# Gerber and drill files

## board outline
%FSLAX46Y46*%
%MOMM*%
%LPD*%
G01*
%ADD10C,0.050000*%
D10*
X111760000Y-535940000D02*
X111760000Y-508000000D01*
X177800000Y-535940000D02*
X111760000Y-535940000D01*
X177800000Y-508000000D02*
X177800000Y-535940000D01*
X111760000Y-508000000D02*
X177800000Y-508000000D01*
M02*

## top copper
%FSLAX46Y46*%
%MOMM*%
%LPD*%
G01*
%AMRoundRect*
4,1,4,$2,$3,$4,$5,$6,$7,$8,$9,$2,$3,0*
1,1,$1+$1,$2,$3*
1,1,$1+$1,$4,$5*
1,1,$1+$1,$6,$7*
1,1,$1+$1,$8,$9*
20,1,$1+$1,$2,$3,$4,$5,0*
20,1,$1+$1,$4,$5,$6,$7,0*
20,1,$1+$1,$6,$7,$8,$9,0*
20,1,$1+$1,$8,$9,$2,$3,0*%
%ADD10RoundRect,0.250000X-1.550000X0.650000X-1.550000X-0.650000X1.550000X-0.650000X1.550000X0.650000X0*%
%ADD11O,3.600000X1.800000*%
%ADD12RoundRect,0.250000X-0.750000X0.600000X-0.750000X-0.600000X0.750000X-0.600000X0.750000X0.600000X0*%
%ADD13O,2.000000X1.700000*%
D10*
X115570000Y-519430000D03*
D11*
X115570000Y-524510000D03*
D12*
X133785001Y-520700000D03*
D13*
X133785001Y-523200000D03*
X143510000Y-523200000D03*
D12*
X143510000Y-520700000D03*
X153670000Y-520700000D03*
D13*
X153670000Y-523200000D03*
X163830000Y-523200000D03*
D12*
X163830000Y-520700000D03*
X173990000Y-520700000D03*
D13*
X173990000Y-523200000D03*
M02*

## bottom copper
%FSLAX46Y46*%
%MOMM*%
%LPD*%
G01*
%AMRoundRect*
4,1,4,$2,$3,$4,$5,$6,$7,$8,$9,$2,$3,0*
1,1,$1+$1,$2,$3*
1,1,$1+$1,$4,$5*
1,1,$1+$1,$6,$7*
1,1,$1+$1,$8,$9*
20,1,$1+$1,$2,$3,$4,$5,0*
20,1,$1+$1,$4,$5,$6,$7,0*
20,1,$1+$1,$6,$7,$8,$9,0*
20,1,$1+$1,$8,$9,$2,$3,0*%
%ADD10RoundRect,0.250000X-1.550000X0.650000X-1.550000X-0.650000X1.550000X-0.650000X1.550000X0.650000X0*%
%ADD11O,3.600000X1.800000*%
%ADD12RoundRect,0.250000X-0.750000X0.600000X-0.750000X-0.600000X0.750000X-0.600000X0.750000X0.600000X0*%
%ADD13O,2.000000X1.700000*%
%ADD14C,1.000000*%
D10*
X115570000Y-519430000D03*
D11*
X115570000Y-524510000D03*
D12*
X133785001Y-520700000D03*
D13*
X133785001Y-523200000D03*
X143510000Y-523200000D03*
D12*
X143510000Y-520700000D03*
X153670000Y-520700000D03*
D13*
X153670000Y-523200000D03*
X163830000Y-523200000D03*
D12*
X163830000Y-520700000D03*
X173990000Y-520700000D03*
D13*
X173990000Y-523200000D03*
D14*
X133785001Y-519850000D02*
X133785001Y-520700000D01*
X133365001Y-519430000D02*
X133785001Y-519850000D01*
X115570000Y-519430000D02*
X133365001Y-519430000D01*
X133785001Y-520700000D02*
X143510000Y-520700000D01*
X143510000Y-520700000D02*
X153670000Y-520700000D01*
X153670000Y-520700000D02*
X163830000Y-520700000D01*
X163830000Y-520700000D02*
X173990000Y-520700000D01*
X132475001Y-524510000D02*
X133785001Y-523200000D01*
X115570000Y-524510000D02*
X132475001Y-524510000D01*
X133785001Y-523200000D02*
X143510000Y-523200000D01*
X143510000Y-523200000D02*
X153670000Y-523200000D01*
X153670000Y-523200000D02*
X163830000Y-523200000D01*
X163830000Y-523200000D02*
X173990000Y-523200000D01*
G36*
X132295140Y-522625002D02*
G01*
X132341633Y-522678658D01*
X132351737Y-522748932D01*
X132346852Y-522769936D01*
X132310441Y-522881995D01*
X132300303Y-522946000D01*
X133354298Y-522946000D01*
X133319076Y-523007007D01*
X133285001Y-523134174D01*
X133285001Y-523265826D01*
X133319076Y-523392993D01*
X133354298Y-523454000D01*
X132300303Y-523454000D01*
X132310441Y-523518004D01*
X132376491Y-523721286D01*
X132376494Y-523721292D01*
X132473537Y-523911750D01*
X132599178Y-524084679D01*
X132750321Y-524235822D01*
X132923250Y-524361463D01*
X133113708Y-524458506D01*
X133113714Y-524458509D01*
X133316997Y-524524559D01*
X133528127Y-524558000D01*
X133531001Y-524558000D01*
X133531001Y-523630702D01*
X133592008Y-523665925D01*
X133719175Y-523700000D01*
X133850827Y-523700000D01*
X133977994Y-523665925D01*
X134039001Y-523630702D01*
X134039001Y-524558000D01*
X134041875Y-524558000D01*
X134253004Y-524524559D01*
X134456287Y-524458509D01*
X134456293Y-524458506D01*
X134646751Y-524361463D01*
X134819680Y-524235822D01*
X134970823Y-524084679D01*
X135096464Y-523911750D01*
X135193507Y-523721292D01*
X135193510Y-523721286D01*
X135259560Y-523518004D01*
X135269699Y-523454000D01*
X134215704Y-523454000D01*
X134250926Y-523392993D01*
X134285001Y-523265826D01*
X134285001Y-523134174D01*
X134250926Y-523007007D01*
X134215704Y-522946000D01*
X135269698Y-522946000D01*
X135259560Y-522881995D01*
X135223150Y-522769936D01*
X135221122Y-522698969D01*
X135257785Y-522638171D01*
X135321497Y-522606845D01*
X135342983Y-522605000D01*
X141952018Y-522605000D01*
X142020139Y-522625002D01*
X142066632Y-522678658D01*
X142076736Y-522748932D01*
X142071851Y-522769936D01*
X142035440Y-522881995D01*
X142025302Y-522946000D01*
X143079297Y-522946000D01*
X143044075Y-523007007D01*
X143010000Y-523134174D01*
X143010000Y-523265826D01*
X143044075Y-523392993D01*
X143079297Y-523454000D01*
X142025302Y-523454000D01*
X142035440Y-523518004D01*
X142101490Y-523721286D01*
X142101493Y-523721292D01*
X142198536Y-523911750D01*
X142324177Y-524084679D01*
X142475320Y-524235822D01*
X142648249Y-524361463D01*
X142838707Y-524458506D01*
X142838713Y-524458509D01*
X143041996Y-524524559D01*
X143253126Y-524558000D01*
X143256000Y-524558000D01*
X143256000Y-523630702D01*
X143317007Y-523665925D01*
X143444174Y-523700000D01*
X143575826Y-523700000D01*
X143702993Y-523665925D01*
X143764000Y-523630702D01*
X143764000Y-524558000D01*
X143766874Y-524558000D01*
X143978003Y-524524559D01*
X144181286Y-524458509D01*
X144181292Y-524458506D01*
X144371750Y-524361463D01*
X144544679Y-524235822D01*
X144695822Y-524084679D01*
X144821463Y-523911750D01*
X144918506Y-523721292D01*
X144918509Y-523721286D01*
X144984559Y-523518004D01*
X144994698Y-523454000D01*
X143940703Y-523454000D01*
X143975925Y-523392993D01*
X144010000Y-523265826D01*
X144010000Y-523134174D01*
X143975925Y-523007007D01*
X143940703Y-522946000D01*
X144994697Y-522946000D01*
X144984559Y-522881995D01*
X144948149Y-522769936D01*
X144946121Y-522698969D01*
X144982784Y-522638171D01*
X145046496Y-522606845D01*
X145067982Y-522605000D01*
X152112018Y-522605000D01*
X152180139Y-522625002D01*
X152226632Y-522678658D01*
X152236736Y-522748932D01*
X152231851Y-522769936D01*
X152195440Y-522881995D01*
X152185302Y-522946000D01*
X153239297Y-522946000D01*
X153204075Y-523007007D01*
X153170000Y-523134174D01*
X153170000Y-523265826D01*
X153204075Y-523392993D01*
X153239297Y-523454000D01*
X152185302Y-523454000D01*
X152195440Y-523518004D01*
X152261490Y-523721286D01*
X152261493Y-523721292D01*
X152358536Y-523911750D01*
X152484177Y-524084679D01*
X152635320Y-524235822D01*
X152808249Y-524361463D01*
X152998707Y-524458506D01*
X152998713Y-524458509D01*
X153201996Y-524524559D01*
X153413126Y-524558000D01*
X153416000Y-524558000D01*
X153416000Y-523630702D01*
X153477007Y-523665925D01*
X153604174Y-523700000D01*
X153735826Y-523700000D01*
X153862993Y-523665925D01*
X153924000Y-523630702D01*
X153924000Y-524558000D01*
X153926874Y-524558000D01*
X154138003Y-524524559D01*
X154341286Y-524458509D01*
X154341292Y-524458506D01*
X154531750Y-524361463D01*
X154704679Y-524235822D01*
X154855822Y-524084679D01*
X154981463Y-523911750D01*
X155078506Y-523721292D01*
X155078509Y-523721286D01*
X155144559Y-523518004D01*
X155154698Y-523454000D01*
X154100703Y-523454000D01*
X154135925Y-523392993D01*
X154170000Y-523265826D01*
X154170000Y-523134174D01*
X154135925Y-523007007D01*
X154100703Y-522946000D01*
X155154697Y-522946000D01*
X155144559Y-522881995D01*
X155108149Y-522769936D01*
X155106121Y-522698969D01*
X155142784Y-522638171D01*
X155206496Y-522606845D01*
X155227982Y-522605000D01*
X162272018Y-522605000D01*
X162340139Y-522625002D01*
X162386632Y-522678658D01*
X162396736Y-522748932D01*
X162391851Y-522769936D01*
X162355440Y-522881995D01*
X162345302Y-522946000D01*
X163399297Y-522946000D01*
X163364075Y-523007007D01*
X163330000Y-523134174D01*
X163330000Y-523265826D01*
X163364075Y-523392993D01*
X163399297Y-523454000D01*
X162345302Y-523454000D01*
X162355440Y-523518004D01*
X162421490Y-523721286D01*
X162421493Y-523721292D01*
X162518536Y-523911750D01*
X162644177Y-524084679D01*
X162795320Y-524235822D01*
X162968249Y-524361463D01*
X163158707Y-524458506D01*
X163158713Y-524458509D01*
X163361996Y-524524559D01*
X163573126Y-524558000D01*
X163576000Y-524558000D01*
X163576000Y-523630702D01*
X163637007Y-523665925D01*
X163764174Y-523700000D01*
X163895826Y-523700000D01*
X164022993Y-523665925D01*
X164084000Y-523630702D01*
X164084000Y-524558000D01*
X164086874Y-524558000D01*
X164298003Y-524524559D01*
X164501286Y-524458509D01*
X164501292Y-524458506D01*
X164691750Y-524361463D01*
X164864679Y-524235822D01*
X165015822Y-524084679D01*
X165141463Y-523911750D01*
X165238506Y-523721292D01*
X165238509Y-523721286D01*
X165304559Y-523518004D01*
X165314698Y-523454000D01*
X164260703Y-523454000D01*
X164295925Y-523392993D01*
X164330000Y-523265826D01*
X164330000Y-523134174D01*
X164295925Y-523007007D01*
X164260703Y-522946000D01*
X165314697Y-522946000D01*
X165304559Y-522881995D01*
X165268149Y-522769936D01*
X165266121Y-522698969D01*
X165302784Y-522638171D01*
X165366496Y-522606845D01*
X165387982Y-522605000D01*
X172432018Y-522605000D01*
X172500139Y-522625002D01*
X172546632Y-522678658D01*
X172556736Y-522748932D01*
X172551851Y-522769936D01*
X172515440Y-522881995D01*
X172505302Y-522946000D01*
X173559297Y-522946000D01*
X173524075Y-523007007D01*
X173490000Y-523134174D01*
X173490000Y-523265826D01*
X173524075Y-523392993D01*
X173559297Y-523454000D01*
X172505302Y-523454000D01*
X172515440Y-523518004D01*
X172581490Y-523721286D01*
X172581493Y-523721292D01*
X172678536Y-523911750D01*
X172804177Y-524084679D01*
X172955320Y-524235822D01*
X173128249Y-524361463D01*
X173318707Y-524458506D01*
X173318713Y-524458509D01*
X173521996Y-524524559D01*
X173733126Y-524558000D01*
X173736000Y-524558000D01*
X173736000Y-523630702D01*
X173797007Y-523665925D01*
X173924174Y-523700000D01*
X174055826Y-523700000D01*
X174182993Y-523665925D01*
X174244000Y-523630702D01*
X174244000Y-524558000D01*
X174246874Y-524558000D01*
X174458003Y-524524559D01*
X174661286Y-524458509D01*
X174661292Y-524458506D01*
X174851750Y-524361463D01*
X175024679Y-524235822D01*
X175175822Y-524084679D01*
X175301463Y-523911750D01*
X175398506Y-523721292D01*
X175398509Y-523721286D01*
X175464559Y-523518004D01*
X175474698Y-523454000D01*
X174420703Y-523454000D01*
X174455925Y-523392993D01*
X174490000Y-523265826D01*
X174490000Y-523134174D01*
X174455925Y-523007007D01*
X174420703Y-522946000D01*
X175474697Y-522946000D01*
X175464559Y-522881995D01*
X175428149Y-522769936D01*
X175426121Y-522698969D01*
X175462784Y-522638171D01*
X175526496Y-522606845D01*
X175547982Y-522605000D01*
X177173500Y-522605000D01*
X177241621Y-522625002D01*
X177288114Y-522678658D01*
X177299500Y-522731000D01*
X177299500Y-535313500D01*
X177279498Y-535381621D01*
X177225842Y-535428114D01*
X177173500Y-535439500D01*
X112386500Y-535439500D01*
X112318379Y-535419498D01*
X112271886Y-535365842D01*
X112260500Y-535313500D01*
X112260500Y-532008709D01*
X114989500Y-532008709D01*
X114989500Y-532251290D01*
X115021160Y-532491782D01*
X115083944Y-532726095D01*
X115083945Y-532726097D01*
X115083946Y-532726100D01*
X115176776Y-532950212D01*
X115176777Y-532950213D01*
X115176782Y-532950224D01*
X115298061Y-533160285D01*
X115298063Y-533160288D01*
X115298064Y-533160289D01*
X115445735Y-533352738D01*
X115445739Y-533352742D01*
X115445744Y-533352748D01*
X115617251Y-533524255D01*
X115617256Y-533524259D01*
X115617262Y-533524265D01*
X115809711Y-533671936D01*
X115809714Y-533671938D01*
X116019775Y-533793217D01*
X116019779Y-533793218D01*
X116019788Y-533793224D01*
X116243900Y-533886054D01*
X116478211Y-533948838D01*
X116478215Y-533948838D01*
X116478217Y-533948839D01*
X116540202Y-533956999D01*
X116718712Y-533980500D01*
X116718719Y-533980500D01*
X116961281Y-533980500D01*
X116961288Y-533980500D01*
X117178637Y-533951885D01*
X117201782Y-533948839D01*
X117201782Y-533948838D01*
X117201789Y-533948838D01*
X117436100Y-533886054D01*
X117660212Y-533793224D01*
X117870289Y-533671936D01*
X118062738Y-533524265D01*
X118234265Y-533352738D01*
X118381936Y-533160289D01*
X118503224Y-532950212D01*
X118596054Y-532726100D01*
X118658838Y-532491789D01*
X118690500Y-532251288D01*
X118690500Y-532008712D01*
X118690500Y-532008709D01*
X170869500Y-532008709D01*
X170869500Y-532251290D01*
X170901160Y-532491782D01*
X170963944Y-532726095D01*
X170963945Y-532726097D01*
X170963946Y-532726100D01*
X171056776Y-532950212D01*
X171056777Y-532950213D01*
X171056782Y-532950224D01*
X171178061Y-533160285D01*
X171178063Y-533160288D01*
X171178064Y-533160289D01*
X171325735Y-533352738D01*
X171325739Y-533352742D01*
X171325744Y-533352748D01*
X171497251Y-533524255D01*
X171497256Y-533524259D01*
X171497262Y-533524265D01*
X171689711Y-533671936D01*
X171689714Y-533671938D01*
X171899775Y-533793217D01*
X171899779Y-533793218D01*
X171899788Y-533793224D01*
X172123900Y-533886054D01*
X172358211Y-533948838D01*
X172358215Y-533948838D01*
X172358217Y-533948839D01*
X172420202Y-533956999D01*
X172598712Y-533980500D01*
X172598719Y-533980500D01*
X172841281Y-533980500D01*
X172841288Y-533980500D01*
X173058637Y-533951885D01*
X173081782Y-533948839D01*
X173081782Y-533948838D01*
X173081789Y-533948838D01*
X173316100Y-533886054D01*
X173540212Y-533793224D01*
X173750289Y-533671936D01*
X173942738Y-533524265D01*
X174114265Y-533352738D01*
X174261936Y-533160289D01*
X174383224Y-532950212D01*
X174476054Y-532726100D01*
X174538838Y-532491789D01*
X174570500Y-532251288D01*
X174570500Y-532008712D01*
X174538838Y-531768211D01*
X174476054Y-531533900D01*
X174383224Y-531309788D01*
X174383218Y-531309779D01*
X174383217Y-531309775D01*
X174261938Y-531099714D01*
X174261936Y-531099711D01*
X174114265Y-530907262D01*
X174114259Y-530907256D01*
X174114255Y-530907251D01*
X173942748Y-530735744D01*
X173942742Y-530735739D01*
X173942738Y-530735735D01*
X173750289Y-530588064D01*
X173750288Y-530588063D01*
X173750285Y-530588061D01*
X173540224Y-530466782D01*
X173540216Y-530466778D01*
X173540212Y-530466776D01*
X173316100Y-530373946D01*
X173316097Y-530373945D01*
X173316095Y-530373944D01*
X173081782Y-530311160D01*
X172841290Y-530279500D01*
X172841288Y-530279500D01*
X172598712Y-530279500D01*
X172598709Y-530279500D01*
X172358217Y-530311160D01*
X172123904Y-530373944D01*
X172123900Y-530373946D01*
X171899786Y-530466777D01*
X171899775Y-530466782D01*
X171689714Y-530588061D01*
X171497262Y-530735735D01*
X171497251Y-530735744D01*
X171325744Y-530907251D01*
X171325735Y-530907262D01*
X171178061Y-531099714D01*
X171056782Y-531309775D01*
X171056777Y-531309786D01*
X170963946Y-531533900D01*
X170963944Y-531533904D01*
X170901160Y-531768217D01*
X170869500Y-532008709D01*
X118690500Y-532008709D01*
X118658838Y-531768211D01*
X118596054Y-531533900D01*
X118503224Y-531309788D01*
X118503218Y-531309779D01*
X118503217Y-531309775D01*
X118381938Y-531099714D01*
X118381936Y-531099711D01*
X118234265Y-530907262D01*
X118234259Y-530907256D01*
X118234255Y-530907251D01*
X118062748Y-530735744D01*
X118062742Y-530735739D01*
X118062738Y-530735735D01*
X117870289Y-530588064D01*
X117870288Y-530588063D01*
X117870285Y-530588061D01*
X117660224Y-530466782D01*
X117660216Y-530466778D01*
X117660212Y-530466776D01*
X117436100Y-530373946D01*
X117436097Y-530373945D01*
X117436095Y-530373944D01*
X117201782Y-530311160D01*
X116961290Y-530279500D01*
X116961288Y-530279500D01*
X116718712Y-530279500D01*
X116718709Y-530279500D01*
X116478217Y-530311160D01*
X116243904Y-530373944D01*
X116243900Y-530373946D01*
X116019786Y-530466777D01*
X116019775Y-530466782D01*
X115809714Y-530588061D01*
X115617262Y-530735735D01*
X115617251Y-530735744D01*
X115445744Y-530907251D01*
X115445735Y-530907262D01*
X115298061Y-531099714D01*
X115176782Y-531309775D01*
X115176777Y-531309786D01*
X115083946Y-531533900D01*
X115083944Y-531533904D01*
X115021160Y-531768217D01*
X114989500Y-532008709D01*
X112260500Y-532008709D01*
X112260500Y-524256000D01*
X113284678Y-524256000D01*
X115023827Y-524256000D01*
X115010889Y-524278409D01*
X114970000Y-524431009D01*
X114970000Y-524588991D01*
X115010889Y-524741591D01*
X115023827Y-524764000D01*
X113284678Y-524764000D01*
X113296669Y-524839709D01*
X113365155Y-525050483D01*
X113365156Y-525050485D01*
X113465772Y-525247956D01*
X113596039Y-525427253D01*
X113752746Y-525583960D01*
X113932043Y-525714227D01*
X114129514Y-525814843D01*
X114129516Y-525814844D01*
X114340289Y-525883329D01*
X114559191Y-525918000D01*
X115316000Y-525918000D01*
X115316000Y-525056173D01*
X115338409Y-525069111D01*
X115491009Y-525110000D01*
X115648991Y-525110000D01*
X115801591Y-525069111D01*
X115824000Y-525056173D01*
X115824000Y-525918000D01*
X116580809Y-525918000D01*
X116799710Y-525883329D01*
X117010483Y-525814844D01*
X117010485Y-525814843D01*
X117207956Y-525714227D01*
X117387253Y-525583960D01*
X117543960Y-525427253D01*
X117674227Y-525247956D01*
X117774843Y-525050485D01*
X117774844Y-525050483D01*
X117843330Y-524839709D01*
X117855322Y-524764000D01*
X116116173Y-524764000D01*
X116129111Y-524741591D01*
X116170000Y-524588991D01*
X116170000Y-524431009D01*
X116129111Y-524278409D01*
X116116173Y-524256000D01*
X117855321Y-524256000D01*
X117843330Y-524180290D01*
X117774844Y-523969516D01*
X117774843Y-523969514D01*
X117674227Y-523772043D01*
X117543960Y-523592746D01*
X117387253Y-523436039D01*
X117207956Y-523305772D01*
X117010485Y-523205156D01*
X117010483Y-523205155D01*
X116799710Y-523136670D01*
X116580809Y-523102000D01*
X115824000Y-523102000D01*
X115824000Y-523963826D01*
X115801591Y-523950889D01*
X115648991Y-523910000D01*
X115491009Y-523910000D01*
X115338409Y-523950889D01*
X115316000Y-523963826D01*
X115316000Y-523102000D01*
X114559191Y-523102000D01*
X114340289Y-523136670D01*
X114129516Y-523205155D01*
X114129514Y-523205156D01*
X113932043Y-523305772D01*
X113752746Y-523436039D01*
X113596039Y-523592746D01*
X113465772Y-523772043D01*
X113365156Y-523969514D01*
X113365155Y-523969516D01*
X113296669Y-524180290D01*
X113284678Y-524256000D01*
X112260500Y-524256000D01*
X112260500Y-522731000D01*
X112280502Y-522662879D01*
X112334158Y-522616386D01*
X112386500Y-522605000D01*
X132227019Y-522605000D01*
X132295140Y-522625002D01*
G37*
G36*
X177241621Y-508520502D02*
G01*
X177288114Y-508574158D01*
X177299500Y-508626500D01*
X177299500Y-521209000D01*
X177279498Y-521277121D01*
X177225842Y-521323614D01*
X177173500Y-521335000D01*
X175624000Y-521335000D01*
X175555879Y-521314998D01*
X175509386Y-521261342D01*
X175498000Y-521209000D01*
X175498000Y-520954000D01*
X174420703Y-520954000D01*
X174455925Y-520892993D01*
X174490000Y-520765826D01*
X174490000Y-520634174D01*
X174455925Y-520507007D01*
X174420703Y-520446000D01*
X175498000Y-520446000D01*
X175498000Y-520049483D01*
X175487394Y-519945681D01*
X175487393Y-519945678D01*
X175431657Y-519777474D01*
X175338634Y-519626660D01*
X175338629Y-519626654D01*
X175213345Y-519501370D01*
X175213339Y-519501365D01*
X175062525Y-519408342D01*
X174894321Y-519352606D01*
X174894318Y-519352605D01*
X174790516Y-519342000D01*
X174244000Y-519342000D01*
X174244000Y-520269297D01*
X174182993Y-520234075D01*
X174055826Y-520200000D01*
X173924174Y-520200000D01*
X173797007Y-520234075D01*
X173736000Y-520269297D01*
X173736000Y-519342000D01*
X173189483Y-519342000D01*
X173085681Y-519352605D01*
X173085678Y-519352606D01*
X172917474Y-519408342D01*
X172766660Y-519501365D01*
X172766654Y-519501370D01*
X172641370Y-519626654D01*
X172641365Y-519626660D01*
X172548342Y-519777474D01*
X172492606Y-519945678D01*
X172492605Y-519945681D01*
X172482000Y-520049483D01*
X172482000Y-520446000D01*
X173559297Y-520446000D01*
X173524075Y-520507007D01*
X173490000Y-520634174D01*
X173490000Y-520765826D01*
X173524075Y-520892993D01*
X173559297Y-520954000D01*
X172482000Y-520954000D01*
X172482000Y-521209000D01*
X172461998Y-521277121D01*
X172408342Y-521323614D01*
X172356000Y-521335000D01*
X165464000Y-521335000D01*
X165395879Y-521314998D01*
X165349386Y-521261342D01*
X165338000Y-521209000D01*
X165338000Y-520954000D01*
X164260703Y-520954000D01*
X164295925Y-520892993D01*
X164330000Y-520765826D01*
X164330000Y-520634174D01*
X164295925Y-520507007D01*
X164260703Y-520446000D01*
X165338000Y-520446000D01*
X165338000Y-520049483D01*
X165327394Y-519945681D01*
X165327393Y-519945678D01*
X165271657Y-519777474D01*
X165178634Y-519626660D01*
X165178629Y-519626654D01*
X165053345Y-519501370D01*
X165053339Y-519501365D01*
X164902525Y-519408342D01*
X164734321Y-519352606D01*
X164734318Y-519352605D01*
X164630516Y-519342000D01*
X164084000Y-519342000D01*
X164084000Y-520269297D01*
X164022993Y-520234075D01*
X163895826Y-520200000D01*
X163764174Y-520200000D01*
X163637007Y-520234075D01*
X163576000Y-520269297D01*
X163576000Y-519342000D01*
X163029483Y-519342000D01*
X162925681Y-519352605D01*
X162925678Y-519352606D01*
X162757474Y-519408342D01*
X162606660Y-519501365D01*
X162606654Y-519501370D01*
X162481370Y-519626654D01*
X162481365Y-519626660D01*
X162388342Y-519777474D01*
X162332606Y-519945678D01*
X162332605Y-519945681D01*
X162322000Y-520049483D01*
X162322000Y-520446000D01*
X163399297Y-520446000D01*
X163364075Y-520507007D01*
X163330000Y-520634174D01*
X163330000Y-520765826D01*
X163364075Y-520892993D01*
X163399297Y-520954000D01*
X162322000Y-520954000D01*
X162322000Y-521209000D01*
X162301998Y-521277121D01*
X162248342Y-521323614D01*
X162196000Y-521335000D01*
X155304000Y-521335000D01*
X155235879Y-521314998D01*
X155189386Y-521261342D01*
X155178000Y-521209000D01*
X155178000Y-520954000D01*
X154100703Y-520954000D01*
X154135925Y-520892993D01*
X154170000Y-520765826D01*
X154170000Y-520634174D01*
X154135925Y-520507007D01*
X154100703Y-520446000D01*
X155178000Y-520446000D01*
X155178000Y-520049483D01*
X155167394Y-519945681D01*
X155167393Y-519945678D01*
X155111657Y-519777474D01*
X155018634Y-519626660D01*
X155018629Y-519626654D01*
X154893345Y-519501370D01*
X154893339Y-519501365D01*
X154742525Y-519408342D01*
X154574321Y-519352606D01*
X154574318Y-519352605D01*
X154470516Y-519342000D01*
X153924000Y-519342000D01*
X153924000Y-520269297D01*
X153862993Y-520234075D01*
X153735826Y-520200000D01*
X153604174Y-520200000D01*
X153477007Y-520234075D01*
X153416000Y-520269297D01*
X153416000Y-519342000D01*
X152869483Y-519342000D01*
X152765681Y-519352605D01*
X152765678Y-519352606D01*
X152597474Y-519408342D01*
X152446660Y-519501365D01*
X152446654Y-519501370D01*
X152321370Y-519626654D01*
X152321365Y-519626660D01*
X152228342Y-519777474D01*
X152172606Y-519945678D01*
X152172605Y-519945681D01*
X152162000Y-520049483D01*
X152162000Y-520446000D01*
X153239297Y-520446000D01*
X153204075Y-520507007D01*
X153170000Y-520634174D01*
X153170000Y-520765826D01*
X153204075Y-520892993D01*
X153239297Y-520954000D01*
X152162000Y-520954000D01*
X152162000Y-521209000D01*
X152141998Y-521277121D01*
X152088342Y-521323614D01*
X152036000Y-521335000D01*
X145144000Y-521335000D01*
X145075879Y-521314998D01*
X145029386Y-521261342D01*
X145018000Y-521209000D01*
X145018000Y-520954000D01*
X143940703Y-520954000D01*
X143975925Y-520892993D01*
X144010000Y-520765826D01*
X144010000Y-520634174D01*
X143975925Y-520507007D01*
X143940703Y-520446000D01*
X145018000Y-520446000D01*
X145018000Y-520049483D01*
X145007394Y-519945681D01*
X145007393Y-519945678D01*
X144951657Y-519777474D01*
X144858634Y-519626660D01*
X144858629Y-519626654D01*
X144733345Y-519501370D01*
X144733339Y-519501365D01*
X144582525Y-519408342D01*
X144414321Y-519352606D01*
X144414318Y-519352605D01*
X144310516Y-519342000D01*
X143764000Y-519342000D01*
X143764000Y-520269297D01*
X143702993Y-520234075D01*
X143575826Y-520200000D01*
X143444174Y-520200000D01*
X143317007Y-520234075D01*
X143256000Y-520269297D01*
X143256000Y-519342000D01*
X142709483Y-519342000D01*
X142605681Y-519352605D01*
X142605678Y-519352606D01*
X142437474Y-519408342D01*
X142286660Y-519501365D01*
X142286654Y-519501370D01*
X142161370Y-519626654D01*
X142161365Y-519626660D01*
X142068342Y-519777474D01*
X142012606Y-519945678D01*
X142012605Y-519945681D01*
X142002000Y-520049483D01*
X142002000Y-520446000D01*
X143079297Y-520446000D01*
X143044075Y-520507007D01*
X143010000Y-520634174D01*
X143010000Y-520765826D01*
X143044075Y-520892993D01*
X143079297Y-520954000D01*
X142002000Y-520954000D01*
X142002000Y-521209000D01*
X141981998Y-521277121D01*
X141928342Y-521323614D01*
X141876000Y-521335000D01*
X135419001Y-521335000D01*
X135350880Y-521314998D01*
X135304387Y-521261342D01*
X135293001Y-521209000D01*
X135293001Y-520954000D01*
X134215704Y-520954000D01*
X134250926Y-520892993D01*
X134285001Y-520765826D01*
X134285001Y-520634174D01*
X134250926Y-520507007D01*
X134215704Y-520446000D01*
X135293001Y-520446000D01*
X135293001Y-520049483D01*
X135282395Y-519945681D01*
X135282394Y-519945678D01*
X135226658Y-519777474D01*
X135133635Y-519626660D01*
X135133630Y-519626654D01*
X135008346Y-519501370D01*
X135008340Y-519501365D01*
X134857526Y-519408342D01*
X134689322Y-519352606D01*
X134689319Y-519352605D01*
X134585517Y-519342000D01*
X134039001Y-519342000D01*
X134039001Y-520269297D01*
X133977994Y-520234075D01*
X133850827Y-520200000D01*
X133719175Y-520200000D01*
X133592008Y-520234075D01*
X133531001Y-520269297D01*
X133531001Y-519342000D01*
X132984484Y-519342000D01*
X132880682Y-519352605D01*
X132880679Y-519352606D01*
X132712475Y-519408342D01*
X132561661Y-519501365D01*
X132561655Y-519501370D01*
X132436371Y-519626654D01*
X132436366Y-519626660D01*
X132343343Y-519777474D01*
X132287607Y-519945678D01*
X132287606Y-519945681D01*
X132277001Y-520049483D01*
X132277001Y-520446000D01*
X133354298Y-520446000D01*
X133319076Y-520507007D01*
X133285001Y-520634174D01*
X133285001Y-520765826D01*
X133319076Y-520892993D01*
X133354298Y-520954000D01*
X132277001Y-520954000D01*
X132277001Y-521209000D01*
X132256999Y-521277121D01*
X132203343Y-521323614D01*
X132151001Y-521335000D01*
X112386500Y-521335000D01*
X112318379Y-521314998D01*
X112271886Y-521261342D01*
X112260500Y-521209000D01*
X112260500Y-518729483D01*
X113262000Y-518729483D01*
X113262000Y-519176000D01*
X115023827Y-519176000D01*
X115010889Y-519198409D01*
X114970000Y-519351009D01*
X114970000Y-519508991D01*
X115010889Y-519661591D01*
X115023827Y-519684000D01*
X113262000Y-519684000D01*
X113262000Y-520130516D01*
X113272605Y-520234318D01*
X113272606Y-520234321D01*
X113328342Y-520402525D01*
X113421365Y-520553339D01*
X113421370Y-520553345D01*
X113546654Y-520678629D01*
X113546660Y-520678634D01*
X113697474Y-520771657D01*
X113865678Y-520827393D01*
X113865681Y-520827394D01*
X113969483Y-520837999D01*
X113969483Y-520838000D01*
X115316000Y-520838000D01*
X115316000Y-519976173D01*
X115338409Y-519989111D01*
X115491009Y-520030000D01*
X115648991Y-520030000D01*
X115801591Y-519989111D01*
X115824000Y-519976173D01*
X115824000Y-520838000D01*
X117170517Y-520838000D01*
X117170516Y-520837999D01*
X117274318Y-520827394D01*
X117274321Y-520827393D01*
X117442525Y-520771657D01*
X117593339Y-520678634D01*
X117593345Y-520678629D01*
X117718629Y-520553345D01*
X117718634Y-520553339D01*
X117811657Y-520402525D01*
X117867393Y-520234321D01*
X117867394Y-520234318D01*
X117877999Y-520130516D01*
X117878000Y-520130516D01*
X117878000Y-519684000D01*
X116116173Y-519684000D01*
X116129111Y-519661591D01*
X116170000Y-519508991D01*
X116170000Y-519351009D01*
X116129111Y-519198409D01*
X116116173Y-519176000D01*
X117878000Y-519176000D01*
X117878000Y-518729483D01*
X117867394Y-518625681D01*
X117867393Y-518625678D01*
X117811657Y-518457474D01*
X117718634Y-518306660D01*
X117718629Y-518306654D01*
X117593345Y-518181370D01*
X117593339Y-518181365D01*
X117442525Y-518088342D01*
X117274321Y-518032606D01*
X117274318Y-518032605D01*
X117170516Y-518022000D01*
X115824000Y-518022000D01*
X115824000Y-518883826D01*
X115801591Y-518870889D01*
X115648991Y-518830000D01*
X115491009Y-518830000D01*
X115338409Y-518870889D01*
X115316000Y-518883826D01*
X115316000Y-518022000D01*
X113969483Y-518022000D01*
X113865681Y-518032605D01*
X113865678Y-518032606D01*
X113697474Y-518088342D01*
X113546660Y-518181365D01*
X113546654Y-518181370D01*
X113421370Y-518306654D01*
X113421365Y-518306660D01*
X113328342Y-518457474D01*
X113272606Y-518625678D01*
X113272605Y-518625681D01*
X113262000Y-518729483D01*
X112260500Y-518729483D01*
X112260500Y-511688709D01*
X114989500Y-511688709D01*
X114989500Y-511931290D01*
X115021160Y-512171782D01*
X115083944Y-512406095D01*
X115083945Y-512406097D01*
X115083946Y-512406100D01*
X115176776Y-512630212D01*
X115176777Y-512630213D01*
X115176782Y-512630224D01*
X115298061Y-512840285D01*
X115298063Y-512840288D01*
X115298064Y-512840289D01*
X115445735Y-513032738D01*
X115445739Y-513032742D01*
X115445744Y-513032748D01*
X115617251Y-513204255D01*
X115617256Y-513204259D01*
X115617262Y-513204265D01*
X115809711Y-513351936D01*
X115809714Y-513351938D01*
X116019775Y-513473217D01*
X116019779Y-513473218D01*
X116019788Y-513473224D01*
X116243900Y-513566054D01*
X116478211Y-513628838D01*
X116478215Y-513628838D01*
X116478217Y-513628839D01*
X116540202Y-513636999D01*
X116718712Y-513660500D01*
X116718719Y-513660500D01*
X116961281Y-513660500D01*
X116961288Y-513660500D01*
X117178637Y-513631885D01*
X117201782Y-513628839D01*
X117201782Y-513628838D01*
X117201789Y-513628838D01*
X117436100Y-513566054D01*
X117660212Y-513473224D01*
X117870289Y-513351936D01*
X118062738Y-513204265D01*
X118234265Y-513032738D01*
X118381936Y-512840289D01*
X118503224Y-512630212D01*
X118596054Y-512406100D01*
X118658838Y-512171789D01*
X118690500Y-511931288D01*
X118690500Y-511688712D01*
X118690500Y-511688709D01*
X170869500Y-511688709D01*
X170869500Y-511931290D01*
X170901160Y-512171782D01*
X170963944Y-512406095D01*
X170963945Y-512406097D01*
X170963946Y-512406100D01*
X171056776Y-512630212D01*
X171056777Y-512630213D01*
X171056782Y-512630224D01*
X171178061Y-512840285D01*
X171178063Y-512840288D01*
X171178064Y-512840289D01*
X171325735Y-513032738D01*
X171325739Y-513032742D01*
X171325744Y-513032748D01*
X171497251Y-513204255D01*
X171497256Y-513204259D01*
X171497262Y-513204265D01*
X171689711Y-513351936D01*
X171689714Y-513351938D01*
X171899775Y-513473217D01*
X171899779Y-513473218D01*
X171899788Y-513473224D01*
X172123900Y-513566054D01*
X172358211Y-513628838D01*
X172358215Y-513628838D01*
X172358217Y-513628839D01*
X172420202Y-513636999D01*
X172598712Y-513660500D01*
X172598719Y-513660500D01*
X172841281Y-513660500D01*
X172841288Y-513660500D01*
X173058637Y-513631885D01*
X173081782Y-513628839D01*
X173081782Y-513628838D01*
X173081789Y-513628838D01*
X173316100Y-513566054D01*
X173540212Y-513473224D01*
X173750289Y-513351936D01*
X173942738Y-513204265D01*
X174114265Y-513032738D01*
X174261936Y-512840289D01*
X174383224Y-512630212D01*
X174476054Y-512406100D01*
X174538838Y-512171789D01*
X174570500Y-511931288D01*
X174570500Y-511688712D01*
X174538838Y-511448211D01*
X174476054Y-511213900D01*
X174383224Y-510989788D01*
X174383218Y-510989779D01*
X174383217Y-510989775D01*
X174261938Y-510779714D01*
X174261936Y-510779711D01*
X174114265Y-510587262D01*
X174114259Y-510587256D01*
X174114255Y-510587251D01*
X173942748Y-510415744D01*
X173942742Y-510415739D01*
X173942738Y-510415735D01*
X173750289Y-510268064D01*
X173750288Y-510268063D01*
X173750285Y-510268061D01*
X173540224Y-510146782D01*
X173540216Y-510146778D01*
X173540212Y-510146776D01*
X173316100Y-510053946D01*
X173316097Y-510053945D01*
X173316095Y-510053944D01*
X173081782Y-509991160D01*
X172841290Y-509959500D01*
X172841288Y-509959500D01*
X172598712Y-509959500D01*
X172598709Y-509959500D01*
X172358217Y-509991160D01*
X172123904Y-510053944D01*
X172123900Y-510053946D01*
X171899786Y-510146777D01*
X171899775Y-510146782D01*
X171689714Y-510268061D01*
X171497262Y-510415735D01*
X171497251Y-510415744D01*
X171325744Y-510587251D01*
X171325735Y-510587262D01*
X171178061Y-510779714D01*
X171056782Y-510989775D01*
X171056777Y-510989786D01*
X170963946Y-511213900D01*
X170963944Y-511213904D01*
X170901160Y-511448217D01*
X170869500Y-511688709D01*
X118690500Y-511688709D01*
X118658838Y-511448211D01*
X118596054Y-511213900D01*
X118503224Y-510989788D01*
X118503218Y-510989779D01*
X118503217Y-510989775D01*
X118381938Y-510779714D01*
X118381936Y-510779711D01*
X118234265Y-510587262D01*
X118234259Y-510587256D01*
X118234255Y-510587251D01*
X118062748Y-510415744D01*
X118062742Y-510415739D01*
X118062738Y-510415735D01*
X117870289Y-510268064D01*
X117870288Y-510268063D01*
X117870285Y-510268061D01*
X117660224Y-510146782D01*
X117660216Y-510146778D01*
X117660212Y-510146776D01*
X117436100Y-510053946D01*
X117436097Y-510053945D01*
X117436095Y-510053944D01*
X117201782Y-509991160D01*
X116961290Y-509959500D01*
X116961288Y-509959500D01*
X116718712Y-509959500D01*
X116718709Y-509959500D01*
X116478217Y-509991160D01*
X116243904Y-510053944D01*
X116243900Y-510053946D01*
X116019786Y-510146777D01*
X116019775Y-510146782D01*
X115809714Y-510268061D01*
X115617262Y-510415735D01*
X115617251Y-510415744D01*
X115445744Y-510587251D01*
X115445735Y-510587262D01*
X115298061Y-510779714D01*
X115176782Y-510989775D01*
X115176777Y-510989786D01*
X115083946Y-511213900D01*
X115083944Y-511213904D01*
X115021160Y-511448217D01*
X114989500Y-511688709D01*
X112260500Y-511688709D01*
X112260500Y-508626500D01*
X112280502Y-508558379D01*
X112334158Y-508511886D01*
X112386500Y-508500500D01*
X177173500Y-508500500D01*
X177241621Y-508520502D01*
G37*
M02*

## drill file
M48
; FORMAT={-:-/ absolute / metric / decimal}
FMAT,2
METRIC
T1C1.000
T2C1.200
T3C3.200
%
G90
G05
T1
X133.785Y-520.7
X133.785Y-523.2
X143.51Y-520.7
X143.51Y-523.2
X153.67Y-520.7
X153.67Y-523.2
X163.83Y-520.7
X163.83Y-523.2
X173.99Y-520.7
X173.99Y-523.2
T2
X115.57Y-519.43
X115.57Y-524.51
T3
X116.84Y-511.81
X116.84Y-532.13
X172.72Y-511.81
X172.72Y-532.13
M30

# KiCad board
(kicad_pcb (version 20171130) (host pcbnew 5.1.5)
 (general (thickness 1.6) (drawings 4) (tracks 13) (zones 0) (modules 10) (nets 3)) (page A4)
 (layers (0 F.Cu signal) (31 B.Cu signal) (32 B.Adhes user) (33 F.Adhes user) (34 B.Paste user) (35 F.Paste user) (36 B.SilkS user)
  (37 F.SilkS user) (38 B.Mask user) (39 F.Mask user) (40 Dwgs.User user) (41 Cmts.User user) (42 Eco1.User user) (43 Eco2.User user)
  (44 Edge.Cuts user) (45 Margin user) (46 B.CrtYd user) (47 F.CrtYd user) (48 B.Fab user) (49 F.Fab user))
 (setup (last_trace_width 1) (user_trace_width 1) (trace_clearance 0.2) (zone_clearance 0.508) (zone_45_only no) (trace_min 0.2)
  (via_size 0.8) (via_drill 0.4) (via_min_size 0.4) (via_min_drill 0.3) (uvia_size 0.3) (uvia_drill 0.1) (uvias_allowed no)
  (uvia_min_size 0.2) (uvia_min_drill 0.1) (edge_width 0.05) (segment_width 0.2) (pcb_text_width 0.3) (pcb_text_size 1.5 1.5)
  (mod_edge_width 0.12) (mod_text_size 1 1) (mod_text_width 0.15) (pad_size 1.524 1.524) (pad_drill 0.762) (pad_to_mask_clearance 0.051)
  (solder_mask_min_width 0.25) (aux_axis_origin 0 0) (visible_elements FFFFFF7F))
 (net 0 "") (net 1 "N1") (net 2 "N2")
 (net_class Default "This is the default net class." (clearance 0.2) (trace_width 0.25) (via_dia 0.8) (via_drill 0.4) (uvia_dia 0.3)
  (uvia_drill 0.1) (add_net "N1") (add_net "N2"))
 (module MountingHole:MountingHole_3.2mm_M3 (layer F.Cu) (at 116.84 511.81)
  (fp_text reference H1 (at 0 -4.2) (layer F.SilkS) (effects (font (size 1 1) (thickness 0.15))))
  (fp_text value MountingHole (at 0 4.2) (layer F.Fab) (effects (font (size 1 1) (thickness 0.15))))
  (pad 1 np_thru_hole circle (at 0 0) (size 3.2 3.2) (drill 3.2) (layers *.Cu *.Mask)))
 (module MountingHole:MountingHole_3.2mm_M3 (layer F.Cu) (at 116.84 532.13)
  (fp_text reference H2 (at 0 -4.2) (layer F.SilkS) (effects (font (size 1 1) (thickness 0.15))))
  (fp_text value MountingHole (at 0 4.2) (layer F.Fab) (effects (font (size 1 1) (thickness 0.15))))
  (pad 1 np_thru_hole circle (at 0 0) (size 3.2 3.2) (drill 3.2) (layers *.Cu *.Mask)))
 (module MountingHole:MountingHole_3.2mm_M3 (layer F.Cu) (at 172.72 511.81)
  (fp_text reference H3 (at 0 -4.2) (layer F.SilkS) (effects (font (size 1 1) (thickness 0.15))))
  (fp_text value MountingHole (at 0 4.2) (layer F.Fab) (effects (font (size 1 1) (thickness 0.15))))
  (pad 1 np_thru_hole circle (at 0 0) (size 3.2 3.2) (drill 3.2) (layers *.Cu *.Mask)))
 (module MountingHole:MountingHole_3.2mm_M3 (layer F.Cu) (at 172.72 532.13)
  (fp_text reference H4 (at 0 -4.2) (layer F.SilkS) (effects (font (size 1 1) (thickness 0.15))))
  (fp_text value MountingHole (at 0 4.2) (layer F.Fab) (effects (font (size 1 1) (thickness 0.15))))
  (pad 1 np_thru_hole circle (at 0 0) (size 3.2 3.2) (drill 3.2) (layers *.Cu *.Mask)))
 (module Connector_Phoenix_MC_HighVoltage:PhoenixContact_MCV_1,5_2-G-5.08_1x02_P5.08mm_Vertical (layer F.Cu) (at 115.57 519.43 270)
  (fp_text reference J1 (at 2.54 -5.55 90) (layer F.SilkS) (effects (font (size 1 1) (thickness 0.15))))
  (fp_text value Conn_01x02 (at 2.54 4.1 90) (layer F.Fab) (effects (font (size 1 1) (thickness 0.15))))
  (pad 1 thru_hole roundrect (at 0 0 270) (size 1.8 3.6) (drill 1.2) (layers *.Cu *.Mask) (roundrect_rratio 0.138889) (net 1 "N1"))
  (pad 2 thru_hole oval (at 5.08 0 270) (size 1.8 3.6) (drill 1.2) (layers *.Cu *.Mask) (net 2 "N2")))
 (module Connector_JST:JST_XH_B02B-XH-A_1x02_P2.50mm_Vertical (layer F.Cu) (at 133.785001 520.7 270)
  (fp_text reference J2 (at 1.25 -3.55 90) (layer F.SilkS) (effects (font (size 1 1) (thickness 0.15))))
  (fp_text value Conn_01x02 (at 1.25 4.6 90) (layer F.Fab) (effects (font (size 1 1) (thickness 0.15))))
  (pad 1 thru_hole roundrect (at 0 0 270) (size 1.7 2) (drill 1) (layers *.Cu *.Mask) (roundrect_rratio 0.147059) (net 1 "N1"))
  (pad 2 thru_hole oval (at 2.5 0 270) (size 1.7 2) (drill 1) (layers *.Cu *.Mask) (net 2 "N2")))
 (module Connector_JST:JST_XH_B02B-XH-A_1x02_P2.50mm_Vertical (layer F.Cu) (at 143.51 520.7 270)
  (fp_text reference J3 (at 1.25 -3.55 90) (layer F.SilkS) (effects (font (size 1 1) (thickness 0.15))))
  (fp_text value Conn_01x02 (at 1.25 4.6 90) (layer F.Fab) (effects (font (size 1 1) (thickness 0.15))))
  (pad 2 thru_hole oval (at 2.5 0 270) (size 1.7 2) (drill 1) (layers *.Cu *.Mask) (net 2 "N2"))
  (pad 1 thru_hole roundrect (at 0 0 270) (size 1.7 2) (drill 1) (layers *.Cu *.Mask) (roundrect_rratio 0.147059) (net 1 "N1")))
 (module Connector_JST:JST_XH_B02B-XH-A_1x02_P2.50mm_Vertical (layer F.Cu) (at 153.67 520.7 270)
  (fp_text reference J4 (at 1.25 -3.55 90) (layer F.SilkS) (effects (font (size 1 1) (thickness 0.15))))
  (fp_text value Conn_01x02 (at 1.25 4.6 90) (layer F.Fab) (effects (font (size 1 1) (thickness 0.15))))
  (pad 1 thru_hole roundrect (at 0 0 270) (size 1.7 2) (drill 1) (layers *.Cu *.Mask) (roundrect_rratio 0.147059) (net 1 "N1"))
  (pad 2 thru_hole oval (at 2.5 0 270) (size 1.7 2) (drill 1) (layers *.Cu *.Mask) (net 2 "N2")))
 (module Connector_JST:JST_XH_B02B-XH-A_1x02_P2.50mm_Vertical (layer F.Cu) (at 163.83 520.7 270)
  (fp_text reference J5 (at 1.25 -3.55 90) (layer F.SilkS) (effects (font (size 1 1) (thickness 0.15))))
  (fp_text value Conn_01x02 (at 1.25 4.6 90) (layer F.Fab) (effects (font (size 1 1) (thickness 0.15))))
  (pad 2 thru_hole oval (at 2.5 0 270) (size 1.7 2) (drill 1) (layers *.Cu *.Mask) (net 2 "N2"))
  (pad 1 thru_hole roundrect (at 0 0 270) (size 1.7 2) (drill 1) (layers *.Cu *.Mask) (roundrect_rratio 0.147059) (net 1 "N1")))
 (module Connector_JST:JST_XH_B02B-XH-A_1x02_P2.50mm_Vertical (layer F.Cu) (at 173.99 520.7 270)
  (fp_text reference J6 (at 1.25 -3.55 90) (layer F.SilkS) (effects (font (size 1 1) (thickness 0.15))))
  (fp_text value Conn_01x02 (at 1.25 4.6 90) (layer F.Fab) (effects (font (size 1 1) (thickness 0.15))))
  (pad 1 thru_hole roundrect (at 0 0 270) (size 1.7 2) (drill 1) (layers *.Cu *.Mask) (roundrect_rratio 0.147059) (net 1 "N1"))
  (pad 2 thru_hole oval (at 2.5 0 270) (size 1.7 2) (drill 1) (layers *.Cu *.Mask) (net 2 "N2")))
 (gr_line (start 111.76 535.94) (end 111.76 508) (layer Edge.Cuts) (width 0.05))
 (gr_line (start 177.8 535.94) (end 111.76 535.94) (layer Edge.Cuts) (width 0.05))
 (gr_line (start 177.8 508) (end 177.8 535.94) (layer Edge.Cuts) (width 0.05))
 (gr_line (start 111.76 508) (end 177.8 508) (layer Edge.Cuts) (width 0.05))
 (segment (start 133.785001 519.85) (end 133.785001 520.7) (width 1) (layer B.Cu) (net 1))
 (segment (start 133.365001 519.43) (end 133.785001 519.85) (width 1) (layer B.Cu) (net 1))
 (segment (start 115.57 519.43) (end 133.365001 519.43) (width 1) (layer B.Cu) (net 1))
 (segment (start 133.785001 520.7) (end 143.51 520.7) (width 1) (layer B.Cu) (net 1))
 (segment (start 143.51 520.7) (end 153.67 520.7) (width 1) (layer B.Cu) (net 1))
 (segment (start 153.67 520.7) (end 163.83 520.7) (width 1) (layer B.Cu) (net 1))
 (segment (start 163.83 520.7) (end 173.99 520.7) (width 1) (layer B.Cu) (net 1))
 (segment (start 132.475001 524.51) (end 133.785001 523.2) (width 1) (layer B.Cu) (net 2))
 (segment (start 115.57 524.51) (end 132.475001 524.51) (width 1) (layer B.Cu) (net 2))
 (segment (start 133.785001 523.2) (end 143.51 523.2) (width 1) (layer B.Cu) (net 2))
 (segment (start 143.51 523.2) (end 153.67 523.2) (width 1) (layer B.Cu) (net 2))
 (segment (start 153.67 523.2) (end 163.83 523.2) (width 1) (layer B.Cu) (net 2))
 (segment (start 163.83 523.2) (end 173.99 523.2) (width 1) (layer B.Cu) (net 2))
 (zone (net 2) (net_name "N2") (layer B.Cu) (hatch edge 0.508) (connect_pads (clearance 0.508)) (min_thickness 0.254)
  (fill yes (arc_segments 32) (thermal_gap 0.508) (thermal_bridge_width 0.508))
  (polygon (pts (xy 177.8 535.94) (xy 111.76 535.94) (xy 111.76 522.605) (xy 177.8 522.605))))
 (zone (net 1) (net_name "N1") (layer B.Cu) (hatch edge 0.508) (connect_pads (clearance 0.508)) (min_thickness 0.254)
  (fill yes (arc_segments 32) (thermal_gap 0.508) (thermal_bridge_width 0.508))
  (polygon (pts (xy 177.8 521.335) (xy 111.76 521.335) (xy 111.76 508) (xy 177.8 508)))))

